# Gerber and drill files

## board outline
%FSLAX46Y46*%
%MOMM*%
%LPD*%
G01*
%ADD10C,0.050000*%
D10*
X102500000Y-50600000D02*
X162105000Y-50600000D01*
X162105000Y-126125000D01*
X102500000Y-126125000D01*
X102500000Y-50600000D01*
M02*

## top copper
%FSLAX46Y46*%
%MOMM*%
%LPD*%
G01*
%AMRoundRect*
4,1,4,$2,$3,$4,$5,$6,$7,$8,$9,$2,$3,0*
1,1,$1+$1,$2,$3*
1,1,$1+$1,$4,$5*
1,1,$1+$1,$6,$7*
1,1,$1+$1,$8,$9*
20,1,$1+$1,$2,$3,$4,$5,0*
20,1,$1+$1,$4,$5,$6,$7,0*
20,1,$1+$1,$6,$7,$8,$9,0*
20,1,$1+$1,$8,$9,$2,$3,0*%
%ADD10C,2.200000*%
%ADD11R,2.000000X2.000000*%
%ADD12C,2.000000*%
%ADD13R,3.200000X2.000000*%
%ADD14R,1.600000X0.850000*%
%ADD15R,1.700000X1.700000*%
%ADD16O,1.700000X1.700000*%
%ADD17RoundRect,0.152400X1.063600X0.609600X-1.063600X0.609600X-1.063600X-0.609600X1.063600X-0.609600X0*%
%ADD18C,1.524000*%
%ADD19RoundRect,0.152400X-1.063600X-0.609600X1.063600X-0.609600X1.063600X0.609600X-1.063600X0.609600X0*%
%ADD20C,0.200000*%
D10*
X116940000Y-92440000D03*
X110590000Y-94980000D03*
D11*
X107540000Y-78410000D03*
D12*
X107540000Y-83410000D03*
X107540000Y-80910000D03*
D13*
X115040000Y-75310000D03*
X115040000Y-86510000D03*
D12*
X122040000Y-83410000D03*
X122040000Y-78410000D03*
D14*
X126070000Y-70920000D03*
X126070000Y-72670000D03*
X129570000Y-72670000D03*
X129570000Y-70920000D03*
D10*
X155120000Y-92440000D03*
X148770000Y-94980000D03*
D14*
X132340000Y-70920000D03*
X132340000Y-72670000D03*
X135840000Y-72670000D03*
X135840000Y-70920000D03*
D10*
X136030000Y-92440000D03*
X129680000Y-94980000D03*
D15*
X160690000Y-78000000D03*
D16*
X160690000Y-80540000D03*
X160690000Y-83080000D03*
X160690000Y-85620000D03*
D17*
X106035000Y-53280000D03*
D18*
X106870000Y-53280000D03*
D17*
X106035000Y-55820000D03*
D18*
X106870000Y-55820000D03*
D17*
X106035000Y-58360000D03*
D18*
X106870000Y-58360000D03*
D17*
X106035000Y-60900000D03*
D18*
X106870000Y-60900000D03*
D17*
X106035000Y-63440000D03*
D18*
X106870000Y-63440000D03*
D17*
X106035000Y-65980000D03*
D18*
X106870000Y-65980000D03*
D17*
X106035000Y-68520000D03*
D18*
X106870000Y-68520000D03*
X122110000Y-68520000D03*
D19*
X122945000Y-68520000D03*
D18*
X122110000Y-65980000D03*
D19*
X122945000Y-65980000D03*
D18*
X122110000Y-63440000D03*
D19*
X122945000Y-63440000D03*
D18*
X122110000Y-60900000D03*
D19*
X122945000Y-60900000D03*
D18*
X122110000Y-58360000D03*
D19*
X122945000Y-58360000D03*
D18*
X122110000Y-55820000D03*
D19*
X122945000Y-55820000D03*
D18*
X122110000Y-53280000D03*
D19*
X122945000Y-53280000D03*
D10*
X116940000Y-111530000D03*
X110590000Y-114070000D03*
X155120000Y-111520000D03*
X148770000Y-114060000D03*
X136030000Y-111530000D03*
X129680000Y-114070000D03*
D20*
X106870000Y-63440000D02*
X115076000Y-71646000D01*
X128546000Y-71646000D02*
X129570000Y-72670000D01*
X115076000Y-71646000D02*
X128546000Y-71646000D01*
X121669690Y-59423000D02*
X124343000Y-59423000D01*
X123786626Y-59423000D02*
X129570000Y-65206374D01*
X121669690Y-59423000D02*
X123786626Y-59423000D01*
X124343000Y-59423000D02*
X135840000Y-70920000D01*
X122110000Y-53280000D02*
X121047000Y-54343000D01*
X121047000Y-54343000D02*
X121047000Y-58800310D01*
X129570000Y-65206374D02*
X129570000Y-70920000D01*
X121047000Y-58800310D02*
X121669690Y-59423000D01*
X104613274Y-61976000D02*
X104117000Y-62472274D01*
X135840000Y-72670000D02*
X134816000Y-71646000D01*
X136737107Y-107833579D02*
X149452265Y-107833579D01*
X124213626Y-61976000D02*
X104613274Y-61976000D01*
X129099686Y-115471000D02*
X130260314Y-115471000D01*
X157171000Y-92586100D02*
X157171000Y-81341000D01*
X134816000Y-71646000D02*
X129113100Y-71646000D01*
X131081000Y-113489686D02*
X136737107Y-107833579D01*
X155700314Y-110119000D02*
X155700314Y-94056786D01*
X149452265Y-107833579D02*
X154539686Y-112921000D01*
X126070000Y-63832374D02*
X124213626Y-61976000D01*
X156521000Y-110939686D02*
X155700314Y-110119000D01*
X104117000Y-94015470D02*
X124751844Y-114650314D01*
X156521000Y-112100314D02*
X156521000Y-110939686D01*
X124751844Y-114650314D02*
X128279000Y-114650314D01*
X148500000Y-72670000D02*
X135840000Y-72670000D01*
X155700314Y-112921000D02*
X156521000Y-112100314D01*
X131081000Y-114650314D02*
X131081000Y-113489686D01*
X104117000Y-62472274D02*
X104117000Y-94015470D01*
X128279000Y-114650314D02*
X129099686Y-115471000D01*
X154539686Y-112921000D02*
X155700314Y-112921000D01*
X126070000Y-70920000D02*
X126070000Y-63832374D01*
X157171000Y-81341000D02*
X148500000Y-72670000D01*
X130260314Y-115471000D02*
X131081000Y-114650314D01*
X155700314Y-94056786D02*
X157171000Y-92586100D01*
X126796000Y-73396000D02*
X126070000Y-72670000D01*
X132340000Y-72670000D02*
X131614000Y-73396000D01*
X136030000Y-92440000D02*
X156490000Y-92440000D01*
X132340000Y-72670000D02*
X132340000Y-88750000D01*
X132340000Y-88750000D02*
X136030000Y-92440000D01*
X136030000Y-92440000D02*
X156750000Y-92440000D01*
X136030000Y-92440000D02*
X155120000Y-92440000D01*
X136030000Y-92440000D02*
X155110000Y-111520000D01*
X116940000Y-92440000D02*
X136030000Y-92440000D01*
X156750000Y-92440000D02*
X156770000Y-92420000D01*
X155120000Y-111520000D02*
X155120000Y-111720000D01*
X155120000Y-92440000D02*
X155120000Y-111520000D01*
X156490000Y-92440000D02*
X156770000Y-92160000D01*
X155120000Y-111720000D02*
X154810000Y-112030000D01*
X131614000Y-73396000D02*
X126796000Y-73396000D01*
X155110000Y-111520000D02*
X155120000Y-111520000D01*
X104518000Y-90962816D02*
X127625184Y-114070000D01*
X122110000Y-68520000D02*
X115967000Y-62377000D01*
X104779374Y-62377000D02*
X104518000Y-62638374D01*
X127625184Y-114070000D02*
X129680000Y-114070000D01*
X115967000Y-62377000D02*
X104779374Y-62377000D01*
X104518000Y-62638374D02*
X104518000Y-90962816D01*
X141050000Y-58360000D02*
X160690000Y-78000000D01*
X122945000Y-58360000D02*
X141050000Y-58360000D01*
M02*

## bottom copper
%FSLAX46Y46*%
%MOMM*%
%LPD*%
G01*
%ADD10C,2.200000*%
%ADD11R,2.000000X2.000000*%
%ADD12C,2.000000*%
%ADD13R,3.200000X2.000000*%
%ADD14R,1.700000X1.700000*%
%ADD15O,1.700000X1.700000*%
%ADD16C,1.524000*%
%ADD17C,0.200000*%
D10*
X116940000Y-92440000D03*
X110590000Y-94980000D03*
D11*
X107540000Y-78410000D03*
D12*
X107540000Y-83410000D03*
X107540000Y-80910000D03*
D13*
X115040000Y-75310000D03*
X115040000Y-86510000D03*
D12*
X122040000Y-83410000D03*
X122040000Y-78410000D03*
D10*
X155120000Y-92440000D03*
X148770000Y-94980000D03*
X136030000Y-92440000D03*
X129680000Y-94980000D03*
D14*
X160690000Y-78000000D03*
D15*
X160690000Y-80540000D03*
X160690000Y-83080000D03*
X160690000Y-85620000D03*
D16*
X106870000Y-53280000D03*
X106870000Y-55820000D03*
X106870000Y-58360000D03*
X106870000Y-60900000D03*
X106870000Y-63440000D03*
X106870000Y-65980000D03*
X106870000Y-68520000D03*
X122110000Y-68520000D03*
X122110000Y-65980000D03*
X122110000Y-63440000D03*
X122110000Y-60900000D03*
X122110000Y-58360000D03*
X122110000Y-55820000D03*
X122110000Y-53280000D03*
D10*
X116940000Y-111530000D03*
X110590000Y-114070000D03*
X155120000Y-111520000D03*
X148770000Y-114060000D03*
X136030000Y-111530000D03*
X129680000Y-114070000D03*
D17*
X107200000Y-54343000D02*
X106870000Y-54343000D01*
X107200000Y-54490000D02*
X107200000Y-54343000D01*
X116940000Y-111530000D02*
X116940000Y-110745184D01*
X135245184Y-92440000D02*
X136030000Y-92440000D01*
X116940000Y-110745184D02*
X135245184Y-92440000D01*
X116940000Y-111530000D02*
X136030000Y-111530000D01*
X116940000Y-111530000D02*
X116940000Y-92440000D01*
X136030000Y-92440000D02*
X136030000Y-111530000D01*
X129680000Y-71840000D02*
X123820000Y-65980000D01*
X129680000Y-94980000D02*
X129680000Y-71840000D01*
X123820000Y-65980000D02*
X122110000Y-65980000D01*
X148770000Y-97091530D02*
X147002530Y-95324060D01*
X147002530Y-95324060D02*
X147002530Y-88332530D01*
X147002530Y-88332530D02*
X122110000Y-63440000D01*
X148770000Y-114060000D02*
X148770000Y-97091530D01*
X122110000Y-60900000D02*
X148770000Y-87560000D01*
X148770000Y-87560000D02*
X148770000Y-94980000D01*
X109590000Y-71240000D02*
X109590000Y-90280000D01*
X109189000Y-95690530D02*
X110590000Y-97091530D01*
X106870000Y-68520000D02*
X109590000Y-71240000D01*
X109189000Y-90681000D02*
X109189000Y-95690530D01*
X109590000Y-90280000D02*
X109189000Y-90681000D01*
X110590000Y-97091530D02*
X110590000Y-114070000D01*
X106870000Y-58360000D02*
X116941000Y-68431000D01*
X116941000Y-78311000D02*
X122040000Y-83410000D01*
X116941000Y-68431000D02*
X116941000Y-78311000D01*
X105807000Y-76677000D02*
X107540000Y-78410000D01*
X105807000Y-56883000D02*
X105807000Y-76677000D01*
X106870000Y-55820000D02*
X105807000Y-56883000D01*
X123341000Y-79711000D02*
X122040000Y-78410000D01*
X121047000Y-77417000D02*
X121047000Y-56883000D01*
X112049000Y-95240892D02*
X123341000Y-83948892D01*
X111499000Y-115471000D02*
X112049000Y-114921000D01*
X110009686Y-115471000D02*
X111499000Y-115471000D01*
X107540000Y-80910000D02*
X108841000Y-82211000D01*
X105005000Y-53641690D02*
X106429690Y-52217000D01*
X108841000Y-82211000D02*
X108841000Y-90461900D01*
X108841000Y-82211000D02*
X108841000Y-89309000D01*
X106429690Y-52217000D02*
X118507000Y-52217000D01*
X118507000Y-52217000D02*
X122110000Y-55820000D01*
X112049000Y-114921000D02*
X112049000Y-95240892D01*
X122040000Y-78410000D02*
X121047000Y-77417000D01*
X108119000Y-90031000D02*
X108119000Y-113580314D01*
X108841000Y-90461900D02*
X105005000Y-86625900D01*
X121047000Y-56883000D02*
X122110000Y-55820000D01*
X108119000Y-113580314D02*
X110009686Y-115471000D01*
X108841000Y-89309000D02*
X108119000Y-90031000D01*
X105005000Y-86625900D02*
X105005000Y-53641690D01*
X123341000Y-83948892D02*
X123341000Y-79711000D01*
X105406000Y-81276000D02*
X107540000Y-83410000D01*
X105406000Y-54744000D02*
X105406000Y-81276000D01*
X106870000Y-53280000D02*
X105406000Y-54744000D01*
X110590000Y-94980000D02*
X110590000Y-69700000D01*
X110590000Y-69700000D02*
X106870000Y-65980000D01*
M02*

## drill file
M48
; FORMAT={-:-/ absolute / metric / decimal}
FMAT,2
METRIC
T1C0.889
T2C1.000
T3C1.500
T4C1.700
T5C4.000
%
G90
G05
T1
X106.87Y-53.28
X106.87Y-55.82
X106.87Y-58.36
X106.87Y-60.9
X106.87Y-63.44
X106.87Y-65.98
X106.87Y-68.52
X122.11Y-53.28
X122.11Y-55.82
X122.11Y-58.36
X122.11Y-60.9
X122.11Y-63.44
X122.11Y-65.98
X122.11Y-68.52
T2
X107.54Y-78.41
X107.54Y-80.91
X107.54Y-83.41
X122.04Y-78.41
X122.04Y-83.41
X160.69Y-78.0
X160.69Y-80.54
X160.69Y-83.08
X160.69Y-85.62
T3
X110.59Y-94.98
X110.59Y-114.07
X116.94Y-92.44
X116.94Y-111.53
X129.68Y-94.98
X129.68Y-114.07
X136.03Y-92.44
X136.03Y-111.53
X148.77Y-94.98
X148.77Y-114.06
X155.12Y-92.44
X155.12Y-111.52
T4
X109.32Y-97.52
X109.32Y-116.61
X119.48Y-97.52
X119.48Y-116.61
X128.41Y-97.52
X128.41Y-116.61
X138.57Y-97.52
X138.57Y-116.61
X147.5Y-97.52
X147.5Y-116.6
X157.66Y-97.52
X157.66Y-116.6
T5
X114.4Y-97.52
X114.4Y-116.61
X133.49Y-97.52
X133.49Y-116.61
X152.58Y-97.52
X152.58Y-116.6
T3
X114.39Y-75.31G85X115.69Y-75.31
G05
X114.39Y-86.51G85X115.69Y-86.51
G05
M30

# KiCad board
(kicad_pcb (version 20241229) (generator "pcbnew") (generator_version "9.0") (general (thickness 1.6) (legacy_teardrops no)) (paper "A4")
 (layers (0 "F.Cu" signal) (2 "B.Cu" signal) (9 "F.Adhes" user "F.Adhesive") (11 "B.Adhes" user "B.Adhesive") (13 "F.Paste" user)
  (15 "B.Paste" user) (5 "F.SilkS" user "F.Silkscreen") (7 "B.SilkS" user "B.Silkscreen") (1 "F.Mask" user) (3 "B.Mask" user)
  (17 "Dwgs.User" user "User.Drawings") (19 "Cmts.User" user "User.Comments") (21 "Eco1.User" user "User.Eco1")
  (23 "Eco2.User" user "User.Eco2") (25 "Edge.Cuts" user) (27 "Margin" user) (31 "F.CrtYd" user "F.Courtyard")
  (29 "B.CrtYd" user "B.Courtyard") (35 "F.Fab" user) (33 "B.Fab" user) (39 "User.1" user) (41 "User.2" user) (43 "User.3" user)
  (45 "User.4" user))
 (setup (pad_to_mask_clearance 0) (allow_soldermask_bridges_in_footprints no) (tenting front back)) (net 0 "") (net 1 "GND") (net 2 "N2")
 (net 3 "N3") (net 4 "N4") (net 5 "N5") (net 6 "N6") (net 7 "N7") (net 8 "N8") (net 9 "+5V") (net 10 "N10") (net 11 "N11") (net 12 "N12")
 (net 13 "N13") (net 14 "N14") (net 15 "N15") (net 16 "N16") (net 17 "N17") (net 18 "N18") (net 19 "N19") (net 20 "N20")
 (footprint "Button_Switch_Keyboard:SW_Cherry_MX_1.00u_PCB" (layer "F.Cu") (at 116.94 92.44)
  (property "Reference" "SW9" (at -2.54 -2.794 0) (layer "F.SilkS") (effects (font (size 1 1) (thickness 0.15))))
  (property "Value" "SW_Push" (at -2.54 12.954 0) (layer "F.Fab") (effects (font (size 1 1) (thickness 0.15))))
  (pad "" np_thru_hole circle (at -7.62 5.08) (size 1.7 1.7) (drill 1.7) (layers "*.Cu" "*.Mask"))
  (pad "" np_thru_hole circle (at -2.54 5.08) (size 4 4) (drill 4) (layers "*.Cu" "*.Mask"))
  (pad "" np_thru_hole circle (at 2.54 5.08) (size 1.7 1.7) (drill 1.7) (layers "*.Cu" "*.Mask"))
  (pad "1" thru_hole circle (at 0 0) (size 2.2 2.2) (drill 1.5) (layers "*.Cu" "*.Mask") (remove_unused_layers no) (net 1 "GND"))
  (pad "2" thru_hole circle (at -6.35 2.54) (size 2.2 2.2) (drill 1.5) (layers "*.Cu" "*.Mask") (remove_unused_layers no) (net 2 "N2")))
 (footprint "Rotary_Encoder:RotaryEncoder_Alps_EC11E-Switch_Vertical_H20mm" (layer "F.Cu") (at 107.54 78.41)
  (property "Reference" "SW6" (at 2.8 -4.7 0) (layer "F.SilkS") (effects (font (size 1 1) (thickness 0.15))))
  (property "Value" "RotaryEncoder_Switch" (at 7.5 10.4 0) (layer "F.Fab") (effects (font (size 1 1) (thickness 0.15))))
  (pad "A" thru_hole rect (at 0 0) (size 2 2) (drill 1) (layers "*.Cu" "*.Mask") (remove_unused_layers no) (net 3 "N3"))
  (pad "B" thru_hole circle (at 0 5) (size 2 2) (drill 1) (layers "*.Cu" "*.Mask") (remove_unused_layers no) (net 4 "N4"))
  (pad "C" thru_hole circle (at 0 2.5) (size 2 2) (drill 1) (layers "*.Cu" "*.Mask") (remove_unused_layers no) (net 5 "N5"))
  (pad "MP" thru_hole rect (at 7.5 -3.1) (size 3.2 2) (drill oval 2.8 1.5) (layers "*.Cu" "*.Mask") (remove_unused_layers no))
  (pad "MP" thru_hole rect (at 7.5 8.1) (size 3.2 2) (drill oval 2.8 1.5) (layers "*.Cu" "*.Mask") (remove_unused_layers no))
  (pad "S1" thru_hole circle (at 14.5 5) (size 2 2) (drill 1) (layers "*.Cu" "*.Mask") (remove_unused_layers no) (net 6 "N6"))
  (pad "S2" thru_hole circle (at 14.5 0) (size 2 2) (drill 1) (layers "*.Cu" "*.Mask") (remove_unused_layers no) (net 5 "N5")))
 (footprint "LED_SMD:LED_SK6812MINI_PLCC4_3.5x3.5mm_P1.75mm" (layer "F.Cu") (at 127.82 71.795)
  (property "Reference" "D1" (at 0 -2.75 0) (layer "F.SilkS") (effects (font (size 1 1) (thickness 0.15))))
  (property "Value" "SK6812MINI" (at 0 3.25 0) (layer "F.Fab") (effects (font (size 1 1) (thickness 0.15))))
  (pad "1" smd rect (at -1.75 -0.875) (size 1.6 0.85) (layers "F.Cu" "F.Mask" "F.Paste") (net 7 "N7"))
  (pad "2" smd rect (at -1.75 0.875) (size 1.6 0.85) (layers "F.Cu" "F.Mask" "F.Paste") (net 1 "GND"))
  (pad "3" smd rect (at 1.75 0.875) (size 1.6 0.85) (layers "F.Cu" "F.Mask" "F.Paste") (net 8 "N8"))
  (pad "4" smd rect (at 1.75 -0.875) (size 1.6 0.85) (layers "F.Cu" "F.Mask" "F.Paste") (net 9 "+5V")))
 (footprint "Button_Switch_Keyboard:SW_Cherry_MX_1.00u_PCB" (layer "F.Cu") (at 155.12 92.44)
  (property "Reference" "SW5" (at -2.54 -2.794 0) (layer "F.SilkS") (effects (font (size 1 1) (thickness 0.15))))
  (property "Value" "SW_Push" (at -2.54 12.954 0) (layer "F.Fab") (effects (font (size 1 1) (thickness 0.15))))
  (pad "" np_thru_hole circle (at -7.62 5.08) (size 1.7 1.7) (drill 1.7) (layers "*.Cu" "*.Mask"))
  (pad "" np_thru_hole circle (at -2.54 5.08) (size 4 4) (drill 4) (layers "*.Cu" "*.Mask"))
  (pad "" np_thru_hole circle (at 2.54 5.08) (size 1.7 1.7) (drill 1.7) (layers "*.Cu" "*.Mask"))
  (pad "1" thru_hole circle (at 0 0) (size 2.2 2.2) (drill 1.5) (layers "*.Cu" "*.Mask") (remove_unused_layers no) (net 1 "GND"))
  (pad "2" thru_hole circle (at -6.35 2.54) (size 2.2 2.2) (drill 1.5) (layers "*.Cu" "*.Mask") (remove_unused_layers no) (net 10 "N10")))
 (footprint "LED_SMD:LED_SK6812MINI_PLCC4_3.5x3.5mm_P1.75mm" (layer "F.Cu") (at 134.09 71.795)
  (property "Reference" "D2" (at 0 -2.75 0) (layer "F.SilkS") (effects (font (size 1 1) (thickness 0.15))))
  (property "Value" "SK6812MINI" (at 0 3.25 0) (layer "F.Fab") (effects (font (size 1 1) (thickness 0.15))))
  (pad "1" smd rect (at -1.75 -0.875) (size 1.6 0.85) (layers "F.Cu" "F.Mask" "F.Paste") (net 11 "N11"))
  (pad "2" smd rect (at -1.75 0.875) (size 1.6 0.85) (layers "F.Cu" "F.Mask" "F.Paste") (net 1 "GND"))
  (pad "3" smd rect (at 1.75 0.875) (size 1.6 0.85) (layers "F.Cu" "F.Mask" "F.Paste") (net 7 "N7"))
  (pad "4" smd rect (at 1.75 -0.875) (size 1.6 0.85) (layers "F.Cu" "F.Mask" "F.Paste") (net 9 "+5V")))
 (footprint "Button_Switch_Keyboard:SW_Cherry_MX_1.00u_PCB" (layer "F.Cu") (at 136.03 92.44)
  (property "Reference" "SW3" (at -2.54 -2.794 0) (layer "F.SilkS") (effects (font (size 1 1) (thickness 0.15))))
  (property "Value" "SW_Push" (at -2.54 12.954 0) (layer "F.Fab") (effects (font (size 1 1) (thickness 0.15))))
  (pad "" np_thru_hole circle (at -7.62 5.08) (size 1.7 1.7) (drill 1.7) (layers "*.Cu" "*.Mask"))
  (pad "" np_thru_hole circle (at -2.54 5.08) (size 4 4) (drill 4) (layers "*.Cu" "*.Mask"))
  (pad "" np_thru_hole circle (at 2.54 5.08) (size 1.7 1.7) (drill 1.7) (layers "*.Cu" "*.Mask"))
  (pad "1" thru_hole circle (at 0 0) (size 2.2 2.2) (drill 1.5) (layers "*.Cu" "*.Mask") (remove_unused_layers no) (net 1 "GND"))
  (pad "2" thru_hole circle (at -6.35 2.54) (size 2.2 2.2) (drill 1.5) (layers "*.Cu" "*.Mask") (remove_unused_layers no) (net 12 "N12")))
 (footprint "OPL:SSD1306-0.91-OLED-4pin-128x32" (layer "F.Cu") (at 124.19 75.81)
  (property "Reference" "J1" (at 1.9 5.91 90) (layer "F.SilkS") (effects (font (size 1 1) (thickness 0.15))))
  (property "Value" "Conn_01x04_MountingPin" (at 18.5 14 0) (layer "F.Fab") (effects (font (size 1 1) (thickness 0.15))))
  (pad "1" thru_hole rect (at 36.5 2.19) (size 1.7 1.7) (drill 1) (layers "*.Cu" "*.Mask") (remove_unused_layers no) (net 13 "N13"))
  (pad "2" thru_hole oval (at 36.5 4.73) (size 1.7 1.7) (drill 1) (layers "*.Cu" "*.Mask") (remove_unused_layers no) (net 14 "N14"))
  (pad "3" thru_hole oval (at 36.5 7.27) (size 1.7 1.7) (drill 1) (layers "*.Cu" "*.Mask") (remove_unused_layers no) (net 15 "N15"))
  (pad "4" thru_hole oval (at 36.5 9.81) (size 1.7 1.7) (drill 1) (layers "*.Cu" "*.Mask") (remove_unused_layers no) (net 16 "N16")))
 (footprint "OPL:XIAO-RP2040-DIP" (layer "F.Cu") (at 114.49 60.9)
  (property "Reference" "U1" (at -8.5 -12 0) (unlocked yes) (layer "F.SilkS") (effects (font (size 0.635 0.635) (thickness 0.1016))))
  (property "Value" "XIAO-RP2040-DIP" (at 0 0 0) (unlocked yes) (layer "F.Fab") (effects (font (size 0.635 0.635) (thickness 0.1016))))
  (pad "1" smd roundrect (at -8.455 -7.62 180) (size 2.432 1.524) (layers "F.Cu" "F.Mask") (roundrect_rratio 0.1) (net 4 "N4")
   (thermal_bridge_angle 45))
  (pad "1" thru_hole circle (at -7.62 -7.62 180) (size 1.524 1.524) (drill 0.889) (layers "*.Cu" "*.Mask") (remove_unused_layers no)
   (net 4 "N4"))
  (pad "2" smd roundrect (at -8.455 -5.08 180) (size 2.432 1.524) (layers "F.Cu" "F.Mask") (roundrect_rratio 0.1) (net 3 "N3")
   (thermal_bridge_angle 45))
  (pad "2" thru_hole circle (at -7.62 -5.08 180) (size 1.524 1.524) (drill 0.889) (layers "*.Cu" "*.Mask") (remove_unused_layers no)
   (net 3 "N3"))
  (pad "3" smd roundrect (at -8.455 -2.54 180) (size 2.432 1.524) (layers "F.Cu" "F.Mask") (roundrect_rratio 0.1) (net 6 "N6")
   (thermal_bridge_angle 45))
  (pad "3" thru_hole circle (at -7.62 -2.54 180) (size 1.524 1.524) (drill 0.889) (layers "*.Cu" "*.Mask") (remove_unused_layers no)
   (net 6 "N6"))
  (pad "4" smd roundrect (at -8.455 0 180) (size 2.432 1.524) (layers "F.Cu" "F.Mask") (roundrect_rratio 0.1) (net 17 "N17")
   (thermal_bridge_angle 45))
  (pad "4" thru_hole circle (at -7.62 0 180) (size 1.524 1.524) (drill 0.889) (layers "*.Cu" "*.Mask") (remove_unused_layers no)
   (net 17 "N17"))
  (pad "5" smd roundrect (at -8.455 2.54 180) (size 2.432 1.524) (layers "F.Cu" "F.Mask") (roundrect_rratio 0.1) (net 8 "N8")
   (thermal_bridge_angle 45))
  (pad "5" thru_hole circle (at -7.62 2.54 180) (size 1.524 1.524) (drill 0.889) (layers "*.Cu" "*.Mask") (remove_unused_layers no)
   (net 8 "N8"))
  (pad "6" smd roundrect (at -8.455 5.08 180) (size 2.432 1.524) (layers "F.Cu" "F.Mask") (roundrect_rratio 0.1) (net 2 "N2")
   (thermal_bridge_angle 45))
  (pad "6" thru_hole circle (at -7.62 5.08 180) (size 1.524 1.524) (drill 0.889) (layers "*.Cu" "*.Mask") (remove_unused_layers no)
   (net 2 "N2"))
  (pad "7" smd roundrect (at -8.455 7.62 180) (size 2.432 1.524) (layers "F.Cu" "F.Mask") (roundrect_rratio 0.1) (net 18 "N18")
   (thermal_bridge_angle 45))
  (pad "7" thru_hole circle (at -7.62 7.62 180) (size 1.524 1.524) (drill 0.889) (layers "*.Cu" "*.Mask") (remove_unused_layers no)
   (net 18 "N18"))
  (pad "8" thru_hole circle (at 7.62 7.62) (size 1.524 1.524) (drill 0.889) (layers "*.Cu" "*.Mask") (remove_unused_layers no)
   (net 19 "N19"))
  (pad "8" smd roundrect (at 8.455 7.62) (size 2.432 1.524) (layers "F.Cu" "F.Mask") (roundrect_rratio 0.1) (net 19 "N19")
   (thermal_bridge_angle 45))
  (pad "9" thru_hole circle (at 7.62 5.08) (size 1.524 1.524) (drill 0.889) (layers "*.Cu" "*.Mask") (remove_unused_layers no)
   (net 12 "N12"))
  (pad "9" smd roundrect (at 8.455 5.08) (size 2.432 1.524) (layers "F.Cu" "F.Mask") (roundrect_rratio 0.1) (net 12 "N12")
   (thermal_bridge_angle 45))
  (pad "10" thru_hole circle (at 7.62 2.54) (size 1.524 1.524) (drill 0.889) (layers "*.Cu" "*.Mask") (remove_unused_layers no)
   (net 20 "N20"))
  (pad "10" smd roundrect (at 8.455 2.54) (size 2.432 1.524) (layers "F.Cu" "F.Mask") (roundrect_rratio 0.1) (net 20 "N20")
   (thermal_bridge_angle 45))
  (pad "11" thru_hole circle (at 7.62 0) (size 1.524 1.524) (drill 0.889) (layers "*.Cu" "*.Mask") (remove_unused_layers no) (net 10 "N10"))
  (pad "11" smd roundrect (at 8.455 0) (size 2.432 1.524) (layers "F.Cu" "F.Mask") (roundrect_rratio 0.1) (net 10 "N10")
   (thermal_bridge_angle 45))
  (pad "12" thru_hole circle (at 7.62 -2.54) (size 1.524 1.524) (drill 0.889) (layers "*.Cu" "*.Mask") (remove_unused_layers no)
   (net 13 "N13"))
  (pad "12" smd roundrect (at 8.455 -2.54) (size 2.432 1.524) (layers "F.Cu" "F.Mask") (roundrect_rratio 0.1) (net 13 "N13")
   (thermal_bridge_angle 45))
  (pad "13" thru_hole circle (at 7.62 -5.08) (size 1.524 1.524) (drill 0.889) (layers "*.Cu" "*.Mask") (remove_unused_layers no)
   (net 5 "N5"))
  (pad "13" smd roundrect (at 8.455 -5.08) (size 2.432 1.524) (layers "F.Cu" "F.Mask") (roundrect_rratio 0.1) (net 5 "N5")
   (thermal_bridge_angle 45))
  (pad "14" thru_hole circle (at 7.62 -7.62) (size 1.524 1.524) (drill 0.889) (layers "*.Cu" "*.Mask") (remove_unused_layers no)
   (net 9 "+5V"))
  (pad "14" smd roundrect (at 8.455 -7.62) (size 2.432 1.524) (layers "F.Cu" "F.Mask") (roundrect_rratio 0.1) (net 9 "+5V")
   (thermal_bridge_angle 45)))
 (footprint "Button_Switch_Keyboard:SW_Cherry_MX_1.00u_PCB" (layer "F.Cu") (at 116.94 111.53)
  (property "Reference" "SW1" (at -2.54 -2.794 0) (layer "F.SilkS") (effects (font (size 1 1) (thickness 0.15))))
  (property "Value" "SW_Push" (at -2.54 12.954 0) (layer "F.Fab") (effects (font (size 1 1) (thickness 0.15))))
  (pad "" np_thru_hole circle (at -7.62 5.08) (size 1.7 1.7) (drill 1.7) (layers "*.Cu" "*.Mask"))
  (pad "" np_thru_hole circle (at -2.54 5.08) (size 4 4) (drill 4) (layers "*.Cu" "*.Mask"))
  (pad "" np_thru_hole circle (at 2.54 5.08) (size 1.7 1.7) (drill 1.7) (layers "*.Cu" "*.Mask"))
  (pad "1" thru_hole circle (at 0 0) (size 2.2 2.2) (drill 1.5) (layers "*.Cu" "*.Mask") (remove_unused_layers no) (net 1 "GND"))
  (pad "2" thru_hole circle (at -6.35 2.54) (size 2.2 2.2) (drill 1.5) (layers "*.Cu" "*.Mask") (remove_unused_layers no) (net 18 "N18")))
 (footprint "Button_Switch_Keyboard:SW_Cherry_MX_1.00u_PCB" (layer "F.Cu") (at 155.12 111.52)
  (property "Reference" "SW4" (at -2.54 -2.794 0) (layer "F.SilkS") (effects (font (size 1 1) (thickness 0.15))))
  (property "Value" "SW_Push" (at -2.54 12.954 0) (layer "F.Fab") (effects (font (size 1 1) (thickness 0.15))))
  (pad "" np_thru_hole circle (at -7.62 5.08) (size 1.7 1.7) (drill 1.7) (layers "*.Cu" "*.Mask"))
  (pad "" np_thru_hole circle (at -2.54 5.08) (size 4 4) (drill 4) (layers "*.Cu" "*.Mask"))
  (pad "" np_thru_hole circle (at 2.54 5.08) (size 1.7 1.7) (drill 1.7) (layers "*.Cu" "*.Mask"))
  (pad "1" thru_hole circle (at 0 0) (size 2.2 2.2) (drill 1.5) (layers "*.Cu" "*.Mask") (remove_unused_layers no) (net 1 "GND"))
  (pad "2" thru_hole circle (at -6.35 2.54) (size 2.2 2.2) (drill 1.5) (layers "*.Cu" "*.Mask") (remove_unused_layers no) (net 20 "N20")))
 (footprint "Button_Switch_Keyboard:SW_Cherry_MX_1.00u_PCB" (layer "F.Cu") (at 136.03 111.53)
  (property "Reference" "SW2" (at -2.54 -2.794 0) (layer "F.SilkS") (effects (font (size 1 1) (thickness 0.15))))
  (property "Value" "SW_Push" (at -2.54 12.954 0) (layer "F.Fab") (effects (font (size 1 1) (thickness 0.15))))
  (pad "" np_thru_hole circle (at -7.62 5.08) (size 1.7 1.7) (drill 1.7) (layers "*.Cu" "*.Mask"))
  (pad "" np_thru_hole circle (at -2.54 5.08) (size 4 4) (drill 4) (layers "*.Cu" "*.Mask"))
  (pad "" np_thru_hole circle (at 2.54 5.08) (size 1.7 1.7) (drill 1.7) (layers "*.Cu" "*.Mask"))
  (pad "1" thru_hole circle (at 0 0) (size 2.2 2.2) (drill 1.5) (layers "*.Cu" "*.Mask") (remove_unused_layers no) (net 1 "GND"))
  (pad "2" thru_hole circle (at -6.35 2.54) (size 2.2 2.2) (drill 1.5) (layers "*.Cu" "*.Mask") (remove_unused_layers no) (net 19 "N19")))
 (gr_rect (start 102.5 50.6) (end 162.105 126.125) (stroke (width 0.05) (type default)) (fill no) (layer "Edge.Cuts"))
 (segment (start 107.2 54.343) (end 106.87 54.343) (width 0.2) (layer "B.Cu") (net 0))
 (segment (start 107.2 54.49) (end 107.2 54.343) (width 0.2) (layer "B.Cu") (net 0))
 (segment (start 106.87 63.44) (end 115.076 71.646) (width 0.2) (layer "F.Cu") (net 8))
 (segment (start 128.546 71.646) (end 129.57 72.67) (width 0.2) (layer "F.Cu") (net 8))
 (segment (start 115.076 71.646) (end 128.546 71.646) (width 0.2) (layer "F.Cu") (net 8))
 (segment (start 121.66969 59.423) (end 124.343 59.423) (width 0.2) (layer "F.Cu") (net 9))
 (segment (start 123.786626 59.423) (end 129.57 65.206374) (width 0.2) (layer "F.Cu") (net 9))
 (segment (start 121.66969 59.423) (end 123.786626 59.423) (width 0.2) (layer "F.Cu") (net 9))
 (segment (start 124.343 59.423) (end 135.84 70.92) (width 0.2) (layer "F.Cu") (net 9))
 (segment (start 122.11 53.28) (end 121.047 54.343) (width 0.2) (layer "F.Cu") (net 9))
 (segment (start 121.047 54.343) (end 121.047 58.80031) (width 0.2) (layer "F.Cu") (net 9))
 (segment (start 129.57 65.206374) (end 129.57 70.92) (width 0.2) (layer "F.Cu") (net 9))
 (segment (start 121.047 58.80031) (end 121.66969 59.423) (width 0.2) (layer "F.Cu") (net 9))
 (segment (start 104.613274 61.976) (end 104.117 62.472274) (width 0.2) (layer "F.Cu") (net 7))
 (segment (start 135.84 72.67) (end 134.816 71.646) (width 0.2) (layer "F.Cu") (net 7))
 (segment (start 136.737107 107.833579) (end 149.452265 107.833579) (width 0.2) (layer "F.Cu") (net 7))
 (segment (start 124.213626 61.976) (end 104.613274 61.976) (width 0.2) (layer "F.Cu") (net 7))
 (segment (start 129.099686 115.471) (end 130.260314 115.471) (width 0.2) (layer "F.Cu") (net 7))
 (segment (start 157.171 92.5861) (end 157.171 81.341) (width 0.2) (layer "F.Cu") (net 7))
 (segment (start 134.816 71.646) (end 129.1131 71.646) (width 0.2) (layer "F.Cu") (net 7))
 (segment (start 131.081 113.489686) (end 136.737107 107.833579) (width 0.2) (layer "F.Cu") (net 7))
 (segment (start 155.700314 110.119) (end 155.700314 94.056786) (width 0.2) (layer "F.Cu") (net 7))
 (segment (start 149.452265 107.833579) (end 154.539686 112.921) (width 0.2) (layer "F.Cu") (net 7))
 (segment (start 126.07 63.832374) (end 124.213626 61.976) (width 0.2) (layer "F.Cu") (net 7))
 (segment (start 156.521 110.939686) (end 155.700314 110.119) (width 0.2) (layer "F.Cu") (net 7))
 (segment (start 104.117 94.01547) (end 124.751844 114.650314) (width 0.2) (layer "F.Cu") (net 7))
 (segment (start 156.521 112.100314) (end 156.521 110.939686) (width 0.2) (layer "F.Cu") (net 7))
 (segment (start 124.751844 114.650314) (end 128.279 114.650314) (width 0.2) (layer "F.Cu") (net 7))
 (segment (start 148.5 72.67) (end 135.84 72.67) (width 0.2) (layer "F.Cu") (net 7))
 (segment (start 155.700314 112.921) (end 156.521 112.100314) (width 0.2) (layer "F.Cu") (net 7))
 (segment (start 131.081 114.650314) (end 131.081 113.489686) (width 0.2) (layer "F.Cu") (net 7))
 (segment (start 104.117 62.472274) (end 104.117 94.01547) (width 0.2) (layer "F.Cu") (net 7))
 (segment (start 128.279 114.650314) (end 129.099686 115.471) (width 0.2) (layer "F.Cu") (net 7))
 (segment (start 154.539686 112.921) (end 155.700314 112.921) (width 0.2) (layer "F.Cu") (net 7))
 (segment (start 126.07 70.92) (end 126.07 63.832374) (width 0.2) (layer "F.Cu") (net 7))
 (segment (start 157.171 81.341) (end 148.5 72.67) (width 0.2) (layer "F.Cu") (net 7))
 (segment (start 130.260314 115.471) (end 131.081 114.650314) (width 0.2) (layer "F.Cu") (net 7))
 (segment (start 155.700314 94.056786) (end 157.171 92.5861) (width 0.2) (layer "F.Cu") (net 7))
 (segment (start 126.796 73.396) (end 126.07 72.67) (width 0.2) (layer "F.Cu") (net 1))
 (segment (start 132.34 72.67) (end 131.614 73.396) (width 0.2) (layer "F.Cu") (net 1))
 (segment (start 136.03 92.44) (end 156.49 92.44) (width 0.2) (layer "F.Cu") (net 1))
 (segment (start 132.34 72.67) (end 132.34 88.75) (width 0.2) (layer "F.Cu") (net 1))
 (segment (start 132.34 88.75) (end 136.03 92.44) (width 0.2) (layer "F.Cu") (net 1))
 (segment (start 136.03 92.44) (end 156.75 92.44) (width 0.2) (layer "F.Cu") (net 1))
 (segment (start 136.03 92.44) (end 155.12 92.44) (width 0.2) (layer "F.Cu") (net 1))
 (segment (start 136.03 92.44) (end 155.11 111.52) (width 0.2) (layer "F.Cu") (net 1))
 (segment (start 116.94 92.44) (end 136.03 92.44) (width 0.2) (layer "F.Cu") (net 1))
 (segment (start 156.75 92.44) (end 156.77 92.42) (width 0.2) (layer "F.Cu") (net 1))
 (segment (start 155.12 111.52) (end 155.12 111.72) (width 0.2) (layer "F.Cu") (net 1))
 (segment (start 155.12 92.44) (end 155.12 111.52) (width 0.2) (layer "F.Cu") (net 1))
 (segment (start 156.49 92.44) (end 156.77 92.16) (width 0.2) (layer "F.Cu") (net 1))
 (segment (start 155.12 111.72) (end 154.81 112.03) (width 0.2) (layer "F.Cu") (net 1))
 (segment (start 131.614 73.396) (end 126.796 73.396) (width 0.2) (layer "F.Cu") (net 1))
 (segment (start 155.11 111.52) (end 155.12 111.52) (width 0.2) (layer "F.Cu") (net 1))
 (segment (start 116.94 111.53) (end 116.94 110.745184) (width 0.2) (layer "B.Cu") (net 1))
 (segment (start 135.245184 92.44) (end 136.03 92.44) (width 0.2) (layer "B.Cu") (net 1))
 (segment (start 116.94 110.745184) (end 135.245184 92.44) (width 0.2) (layer "B.Cu") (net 1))
 (segment (start 116.94 111.53) (end 136.03 111.53) (width 0.2) (layer "B.Cu") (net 1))
 (segment (start 116.94 111.53) (end 116.94 92.44) (width 0.2) (layer "B.Cu") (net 1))
 (segment (start 136.03 92.44) (end 136.03 111.53) (width 0.2) (layer "B.Cu") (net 1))
 (segment (start 104.518 90.962816) (end 127.625184 114.07) (width 0.2) (layer "F.Cu") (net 19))
 (segment (start 122.11 68.52) (end 115.967 62.377) (width 0.2) (layer "F.Cu") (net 19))
 (segment (start 104.779374 62.377) (end 104.518 62.638374) (width 0.2) (layer "F.Cu") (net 19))
 (segment (start 127.625184 114.07) (end 129.68 114.07) (width 0.2) (layer "F.Cu") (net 19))
 (segment (start 115.967 62.377) (end 104.779374 62.377) (width 0.2) (layer "F.Cu") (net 19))
 (segment (start 104.518 62.638374) (end 104.518 90.962816) (width 0.2) (layer "F.Cu") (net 19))
 (segment (start 129.68 71.84) (end 123.82 65.98) (width 0.2) (layer "B.Cu") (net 12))
 (segment (start 129.68 94.98) (end 129.68 71.84) (width 0.2) (layer "B.Cu") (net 12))
 (segment (start 123.82 65.98) (end 122.11 65.98) (width 0.2) (layer "B.Cu") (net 12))
 (segment (start 148.77 97.09153) (end 147.00253 95.32406) (width 0.2) (layer "B.Cu") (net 20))
 (segment (start 147.00253 95.32406) (end 147.00253 88.33253) (width 0.2) (layer "B.Cu") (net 20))
 (segment (start 147.00253 88.33253) (end 122.11 63.44) (width 0.2) (layer "B.Cu") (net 20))
 (segment (start 148.77 114.06) (end 148.77 97.09153) (width 0.2) (layer "B.Cu") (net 20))
 (segment (start 122.11 60.9) (end 148.77 87.56) (width 0.2) (layer "B.Cu") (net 10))
 (segment (start 148.77 87.56) (end 148.77 94.98) (width 0.2) (layer "B.Cu") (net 10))
 (segment (start 109.59 71.24) (end 109.59 90.28) (width 0.2) (layer "B.Cu") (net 18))
 (segment (start 109.189 95.69053) (end 110.59 97.09153) (width 0.2) (layer "B.Cu") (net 18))
 (segment (start 106.87 68.52) (end 109.59 71.24) (width 0.2) (layer "B.Cu") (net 18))
 (segment (start 109.189 90.681) (end 109.189 95.69053) (width 0.2) (layer "B.Cu") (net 18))
 (segment (start 109.59 90.28) (end 109.189 90.681) (width 0.2) (layer "B.Cu") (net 18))
 (segment (start 110.59 97.09153) (end 110.59 114.07) (width 0.2) (layer "B.Cu") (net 18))
 (segment (start 141.05 58.36) (end 160.69 78) (width 0.2) (layer "F.Cu") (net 13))
 (segment (start 122.945 58.36) (end 141.05 58.36) (width 0.2) (layer "F.Cu") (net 13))
 (segment (start 106.87 58.36) (end 116.941 68.431) (width 0.2) (layer "B.Cu") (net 6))
 (segment (start 116.941 78.311) (end 122.04 83.41) (width 0.2) (layer "B.Cu") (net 6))
 (segment (start 116.941 68.431) (end 116.941 78.311) (width 0.2) (layer "B.Cu") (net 6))
 (segment (start 105.807 76.677) (end 107.54 78.41) (width 0.2) (layer "B.Cu") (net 3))
 (segment (start 105.807 56.883) (end 105.807 76.677) (width 0.2) (layer "B.Cu") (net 3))
 (segment (start 106.87 55.82) (end 105.807 56.883) (width 0.2) (layer "B.Cu") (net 3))
 (segment (start 123.341 79.711) (end 122.04 78.41) (width 0.2) (layer "B.Cu") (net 5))
 (segment (start 121.047 77.417) (end 121.047 56.883) (width 0.2) (layer "B.Cu") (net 5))
 (segment (start 112.049 95.240892) (end 123.341 83.948892) (width 0.2) (layer "B.Cu") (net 5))
 (segment (start 111.499 115.471) (end 112.049 114.921) (width 0.2) (layer "B.Cu") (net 5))
 (segment (start 110.009686 115.471) (end 111.499 115.471) (width 0.2) (layer "B.Cu") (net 5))
 (segment (start 107.54 80.91) (end 108.841 82.211) (width 0.2) (layer "B.Cu") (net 5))
 (segment (start 105.005 53.64169) (end 106.42969 52.217) (width 0.2) (layer "B.Cu") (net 5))
 (segment (start 108.841 82.211) (end 108.841 90.4619) (width 0.2) (layer "B.Cu") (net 5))
 (segment (start 108.841 82.211) (end 108.841 89.309) (width 0.2) (layer "B.Cu") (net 5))
 (segment (start 106.42969 52.217) (end 118.507 52.217) (width 0.2) (layer "B.Cu") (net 5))
 (segment (start 118.507 52.217) (end 122.11 55.82) (width 0.2) (layer "B.Cu") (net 5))
 (segment (start 112.049 114.921) (end 112.049 95.240892) (width 0.2) (layer "B.Cu") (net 5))
 (segment (start 122.04 78.41) (end 121.047 77.417) (width 0.2) (layer "B.Cu") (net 5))
 (segment (start 108.119 90.031) (end 108.119 113.580314) (width 0.2) (layer "B.Cu") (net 5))
 (segment (start 108.841 90.4619) (end 105.005 86.6259) (width 0.2) (layer "B.Cu") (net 5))
 (segment (start 121.047 56.883) (end 122.11 55.82) (width 0.2) (layer "B.Cu") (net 5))
 (segment (start 108.119 113.580314) (end 110.009686 115.471) (width 0.2) (layer "B.Cu") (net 5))
 (segment (start 108.841 89.309) (end 108.119 90.031) (width 0.2) (layer "B.Cu") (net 5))
 (segment (start 105.005 86.6259) (end 105.005 53.64169) (width 0.2) (layer "B.Cu") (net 5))
 (segment (start 123.341 83.948892) (end 123.341 79.711) (width 0.2) (layer "B.Cu") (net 5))
 (segment (start 105.406 81.276) (end 107.54 83.41) (width 0.2) (layer "B.Cu") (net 4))
 (segment (start 105.406 54.744) (end 105.406 81.276) (width 0.2) (layer "B.Cu") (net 4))
 (segment (start 106.87 53.28) (end 105.406 54.744) (width 0.2) (layer "B.Cu") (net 4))
 (segment (start 110.59 94.98) (end 110.59 69.7) (width 0.2) (layer "B.Cu") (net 2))
 (segment (start 110.59 69.7) (end 106.87 65.98) (width 0.2) (layer "B.Cu") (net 2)))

